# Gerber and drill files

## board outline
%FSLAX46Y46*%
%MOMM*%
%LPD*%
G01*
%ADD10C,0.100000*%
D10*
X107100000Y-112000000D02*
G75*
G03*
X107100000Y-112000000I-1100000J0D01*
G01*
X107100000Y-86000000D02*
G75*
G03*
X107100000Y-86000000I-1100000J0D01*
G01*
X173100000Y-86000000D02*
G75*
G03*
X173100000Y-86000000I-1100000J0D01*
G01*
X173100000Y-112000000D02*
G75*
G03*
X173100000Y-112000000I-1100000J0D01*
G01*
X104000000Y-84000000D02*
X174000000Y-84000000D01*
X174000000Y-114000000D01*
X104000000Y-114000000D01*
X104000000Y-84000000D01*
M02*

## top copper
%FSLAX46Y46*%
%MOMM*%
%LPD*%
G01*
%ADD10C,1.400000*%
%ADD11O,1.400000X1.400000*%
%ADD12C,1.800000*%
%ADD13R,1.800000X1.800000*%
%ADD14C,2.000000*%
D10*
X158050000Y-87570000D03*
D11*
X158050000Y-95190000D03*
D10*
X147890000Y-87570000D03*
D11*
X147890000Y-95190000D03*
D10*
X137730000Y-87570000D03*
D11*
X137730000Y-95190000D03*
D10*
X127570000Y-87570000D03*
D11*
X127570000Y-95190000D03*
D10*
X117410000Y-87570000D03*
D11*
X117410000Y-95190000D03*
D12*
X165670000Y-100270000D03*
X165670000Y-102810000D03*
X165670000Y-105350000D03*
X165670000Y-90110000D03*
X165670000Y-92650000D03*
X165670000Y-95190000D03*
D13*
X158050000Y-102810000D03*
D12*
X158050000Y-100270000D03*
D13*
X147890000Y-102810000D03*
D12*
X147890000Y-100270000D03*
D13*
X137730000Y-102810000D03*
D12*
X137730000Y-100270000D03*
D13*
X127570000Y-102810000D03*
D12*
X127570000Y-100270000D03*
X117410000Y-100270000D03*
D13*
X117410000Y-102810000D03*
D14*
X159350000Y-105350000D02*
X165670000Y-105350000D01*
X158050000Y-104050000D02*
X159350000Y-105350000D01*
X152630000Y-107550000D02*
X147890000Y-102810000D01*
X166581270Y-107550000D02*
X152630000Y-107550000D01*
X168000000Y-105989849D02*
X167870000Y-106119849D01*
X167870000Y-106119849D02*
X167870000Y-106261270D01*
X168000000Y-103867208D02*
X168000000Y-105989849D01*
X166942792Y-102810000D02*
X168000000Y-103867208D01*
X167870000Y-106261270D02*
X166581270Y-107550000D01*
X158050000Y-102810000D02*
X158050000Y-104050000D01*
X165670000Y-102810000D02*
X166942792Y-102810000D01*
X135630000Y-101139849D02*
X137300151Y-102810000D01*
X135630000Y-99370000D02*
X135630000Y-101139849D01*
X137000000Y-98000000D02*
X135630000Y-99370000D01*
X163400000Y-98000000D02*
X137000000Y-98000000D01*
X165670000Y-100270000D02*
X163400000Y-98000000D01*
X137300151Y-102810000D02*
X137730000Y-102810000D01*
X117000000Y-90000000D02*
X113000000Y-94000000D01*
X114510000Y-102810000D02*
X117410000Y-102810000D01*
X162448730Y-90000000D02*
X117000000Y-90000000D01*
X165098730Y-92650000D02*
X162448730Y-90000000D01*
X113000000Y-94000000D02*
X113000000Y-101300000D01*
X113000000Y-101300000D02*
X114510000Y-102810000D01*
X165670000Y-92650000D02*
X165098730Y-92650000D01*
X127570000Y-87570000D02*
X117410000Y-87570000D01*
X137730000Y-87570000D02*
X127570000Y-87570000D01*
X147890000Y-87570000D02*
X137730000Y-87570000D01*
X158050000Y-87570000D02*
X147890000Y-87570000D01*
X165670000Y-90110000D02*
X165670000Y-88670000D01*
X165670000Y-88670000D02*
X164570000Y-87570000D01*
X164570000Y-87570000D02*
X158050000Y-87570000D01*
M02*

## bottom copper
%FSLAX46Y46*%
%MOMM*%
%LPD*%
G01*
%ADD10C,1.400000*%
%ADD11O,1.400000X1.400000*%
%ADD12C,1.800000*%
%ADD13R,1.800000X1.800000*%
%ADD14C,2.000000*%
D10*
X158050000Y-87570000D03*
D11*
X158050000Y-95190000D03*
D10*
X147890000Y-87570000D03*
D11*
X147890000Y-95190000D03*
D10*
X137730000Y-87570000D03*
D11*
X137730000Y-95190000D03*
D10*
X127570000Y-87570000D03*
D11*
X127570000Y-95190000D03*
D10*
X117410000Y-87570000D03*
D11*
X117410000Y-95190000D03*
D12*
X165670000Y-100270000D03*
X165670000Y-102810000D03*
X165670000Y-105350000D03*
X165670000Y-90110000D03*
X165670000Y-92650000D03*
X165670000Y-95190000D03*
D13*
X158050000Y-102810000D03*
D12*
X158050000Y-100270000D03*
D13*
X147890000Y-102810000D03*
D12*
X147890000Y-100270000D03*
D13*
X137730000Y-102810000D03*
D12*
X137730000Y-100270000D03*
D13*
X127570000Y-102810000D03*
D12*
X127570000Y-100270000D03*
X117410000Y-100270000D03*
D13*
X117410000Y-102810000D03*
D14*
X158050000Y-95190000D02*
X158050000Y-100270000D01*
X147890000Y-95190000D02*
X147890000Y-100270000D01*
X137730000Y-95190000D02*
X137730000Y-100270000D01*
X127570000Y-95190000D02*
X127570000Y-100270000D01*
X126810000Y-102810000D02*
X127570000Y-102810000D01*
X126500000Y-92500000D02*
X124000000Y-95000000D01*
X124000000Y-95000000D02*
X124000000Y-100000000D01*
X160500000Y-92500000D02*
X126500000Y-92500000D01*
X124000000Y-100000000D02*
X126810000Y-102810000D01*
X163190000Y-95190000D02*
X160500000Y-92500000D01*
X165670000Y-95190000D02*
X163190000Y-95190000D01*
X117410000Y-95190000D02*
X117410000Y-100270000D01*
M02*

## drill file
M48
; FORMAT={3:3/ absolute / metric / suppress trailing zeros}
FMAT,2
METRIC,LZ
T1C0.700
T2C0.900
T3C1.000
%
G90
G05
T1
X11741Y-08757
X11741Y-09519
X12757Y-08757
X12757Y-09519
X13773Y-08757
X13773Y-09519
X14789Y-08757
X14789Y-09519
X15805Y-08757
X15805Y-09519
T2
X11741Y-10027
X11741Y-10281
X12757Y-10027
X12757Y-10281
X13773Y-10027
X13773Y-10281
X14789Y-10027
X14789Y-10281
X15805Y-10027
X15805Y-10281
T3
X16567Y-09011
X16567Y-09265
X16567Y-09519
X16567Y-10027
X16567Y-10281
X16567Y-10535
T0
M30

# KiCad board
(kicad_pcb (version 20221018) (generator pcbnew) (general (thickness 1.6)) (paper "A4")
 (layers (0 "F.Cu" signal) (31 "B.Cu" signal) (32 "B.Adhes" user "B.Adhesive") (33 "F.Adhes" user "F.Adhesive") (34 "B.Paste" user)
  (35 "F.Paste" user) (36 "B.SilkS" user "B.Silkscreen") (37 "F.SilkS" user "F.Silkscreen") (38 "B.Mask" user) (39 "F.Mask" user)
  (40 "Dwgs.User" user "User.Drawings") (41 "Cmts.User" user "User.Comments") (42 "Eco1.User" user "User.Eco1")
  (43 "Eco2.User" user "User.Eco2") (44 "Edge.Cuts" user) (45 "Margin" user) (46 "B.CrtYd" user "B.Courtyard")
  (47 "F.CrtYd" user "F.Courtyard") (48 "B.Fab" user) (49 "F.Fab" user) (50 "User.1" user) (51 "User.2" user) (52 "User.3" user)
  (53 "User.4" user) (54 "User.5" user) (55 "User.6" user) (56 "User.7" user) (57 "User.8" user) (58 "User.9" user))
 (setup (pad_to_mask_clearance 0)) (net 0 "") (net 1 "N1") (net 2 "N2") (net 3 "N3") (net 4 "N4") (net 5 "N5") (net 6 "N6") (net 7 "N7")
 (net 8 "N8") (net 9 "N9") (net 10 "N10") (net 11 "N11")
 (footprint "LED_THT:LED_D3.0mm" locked (layer "F.Cu") (at 117.41 102.81 90)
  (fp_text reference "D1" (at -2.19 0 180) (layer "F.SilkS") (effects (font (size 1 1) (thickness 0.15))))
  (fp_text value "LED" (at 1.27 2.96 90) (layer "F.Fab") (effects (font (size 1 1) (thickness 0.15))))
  (pad "1" thru_hole rect locked (at 0 0 90) (size 1.8 1.8) (drill 0.9) (layers "*.Cu" "*.Mask") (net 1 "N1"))
  (pad "2" thru_hole circle locked (at 2.54 0 90) (size 1.8 1.8) (drill 0.9) (layers "*.Cu" "*.Mask") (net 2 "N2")))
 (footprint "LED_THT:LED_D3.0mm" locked (layer "F.Cu") (at 158.05 102.81 90)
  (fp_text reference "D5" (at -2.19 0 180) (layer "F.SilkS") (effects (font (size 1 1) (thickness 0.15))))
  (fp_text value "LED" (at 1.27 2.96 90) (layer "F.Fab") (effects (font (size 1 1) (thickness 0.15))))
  (pad "1" thru_hole rect locked (at 0 0 90) (size 1.8 1.8) (drill 0.9) (layers "*.Cu" "*.Mask") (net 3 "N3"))
  (pad "2" thru_hole circle locked (at 2.54 0 90) (size 1.8 1.8) (drill 0.9) (layers "*.Cu" "*.Mask") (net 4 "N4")))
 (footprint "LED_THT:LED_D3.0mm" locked (layer "F.Cu") (at 127.57 102.81 90)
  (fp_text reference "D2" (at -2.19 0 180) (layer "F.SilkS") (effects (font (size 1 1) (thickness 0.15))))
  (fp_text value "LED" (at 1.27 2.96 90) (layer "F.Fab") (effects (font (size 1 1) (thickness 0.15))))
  (pad "1" thru_hole rect locked (at 0 0 90) (size 1.8 1.8) (drill 0.9) (layers "*.Cu" "*.Mask") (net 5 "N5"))
  (pad "2" thru_hole circle locked (at 2.54 0 90) (size 1.8 1.8) (drill 0.9) (layers "*.Cu" "*.Mask") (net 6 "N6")))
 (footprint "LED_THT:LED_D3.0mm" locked (layer "F.Cu") (at 137.73 102.81 90)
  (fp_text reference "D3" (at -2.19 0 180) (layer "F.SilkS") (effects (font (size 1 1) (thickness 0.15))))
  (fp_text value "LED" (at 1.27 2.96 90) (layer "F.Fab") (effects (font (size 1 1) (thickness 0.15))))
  (pad "1" thru_hole rect locked (at 0 0 90) (size 1.8 1.8) (drill 0.9) (layers "*.Cu" "*.Mask") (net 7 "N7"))
  (pad "2" thru_hole circle locked (at 2.54 0 90) (size 1.8 1.8) (drill 0.9) (layers "*.Cu" "*.Mask") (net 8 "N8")))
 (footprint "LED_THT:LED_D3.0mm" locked (layer "F.Cu") (at 147.89 102.81 90)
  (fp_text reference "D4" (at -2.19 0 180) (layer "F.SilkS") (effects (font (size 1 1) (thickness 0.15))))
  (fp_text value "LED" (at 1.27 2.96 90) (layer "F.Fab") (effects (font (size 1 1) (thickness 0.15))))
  (pad "1" thru_hole rect locked (at 0 0 90) (size 1.8 1.8) (drill 0.9) (layers "*.Cu" "*.Mask") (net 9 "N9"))
  (pad "2" thru_hole circle locked (at 2.54 0 90) (size 1.8 1.8) (drill 0.9) (layers "*.Cu" "*.Mask") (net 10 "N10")))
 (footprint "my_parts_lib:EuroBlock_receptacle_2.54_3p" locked (layer "B.Cu") (at 165.67 102.81 90)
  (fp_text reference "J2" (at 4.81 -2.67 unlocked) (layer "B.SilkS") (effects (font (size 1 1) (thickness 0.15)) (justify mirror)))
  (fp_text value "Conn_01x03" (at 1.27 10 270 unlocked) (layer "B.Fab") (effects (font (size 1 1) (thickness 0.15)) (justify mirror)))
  (pad "1" thru_hole circle locked (at 2.54 0 90) (size 1.8 1.8) (drill 1) (layers "*.Cu" "*.Mask") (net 7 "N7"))
  (pad "2" thru_hole circle locked (at 0 0 90) (size 1.8 1.8) (drill 1) (layers "*.Cu" "*.Mask") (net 9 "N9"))
  (pad "3" thru_hole circle locked (at -2.54 0 90) (size 1.8 1.8) (drill 1) (layers "*.Cu" "*.Mask") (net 3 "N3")))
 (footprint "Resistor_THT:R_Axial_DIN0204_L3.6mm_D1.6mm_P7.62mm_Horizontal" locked (layer "B.Cu") (at 147.89 87.57 -90)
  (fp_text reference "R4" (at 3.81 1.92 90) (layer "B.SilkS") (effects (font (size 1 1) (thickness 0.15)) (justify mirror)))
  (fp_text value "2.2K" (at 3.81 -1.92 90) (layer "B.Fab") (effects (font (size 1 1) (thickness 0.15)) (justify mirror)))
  (pad "1" thru_hole circle locked (at 0 0 270) (size 1.4 1.4) (drill 0.7) (layers "*.Cu" "*.Mask") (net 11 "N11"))
  (pad "2" thru_hole oval locked (at 7.62 0 270) (size 1.4 1.4) (drill 0.7) (layers "*.Cu" "*.Mask") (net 10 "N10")))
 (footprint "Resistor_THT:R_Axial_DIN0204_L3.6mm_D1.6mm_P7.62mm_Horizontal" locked (layer "B.Cu") (at 127.57 87.57 -90)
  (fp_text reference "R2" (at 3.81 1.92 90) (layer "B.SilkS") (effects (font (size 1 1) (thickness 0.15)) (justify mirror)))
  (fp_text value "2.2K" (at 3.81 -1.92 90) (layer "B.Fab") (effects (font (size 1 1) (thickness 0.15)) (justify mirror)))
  (pad "1" thru_hole circle locked (at 0 0 270) (size 1.4 1.4) (drill 0.7) (layers "*.Cu" "*.Mask") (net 11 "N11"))
  (pad "2" thru_hole oval locked (at 7.62 0 270) (size 1.4 1.4) (drill 0.7) (layers "*.Cu" "*.Mask") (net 6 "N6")))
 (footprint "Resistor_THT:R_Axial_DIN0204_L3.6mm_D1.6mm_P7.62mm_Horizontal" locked (layer "B.Cu") (at 158.05 87.57 -90)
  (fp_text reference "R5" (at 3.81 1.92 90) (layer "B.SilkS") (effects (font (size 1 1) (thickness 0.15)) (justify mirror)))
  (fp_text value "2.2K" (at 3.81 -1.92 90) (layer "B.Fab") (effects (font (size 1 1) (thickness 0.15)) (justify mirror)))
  (pad "1" thru_hole circle locked (at 0 0 270) (size 1.4 1.4) (drill 0.7) (layers "*.Cu" "*.Mask") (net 11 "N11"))
  (pad "2" thru_hole oval locked (at 7.62 0 270) (size 1.4 1.4) (drill 0.7) (layers "*.Cu" "*.Mask") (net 4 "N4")))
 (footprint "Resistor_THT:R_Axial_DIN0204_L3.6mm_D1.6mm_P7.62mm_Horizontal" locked (layer "B.Cu") (at 117.41 87.57 -90)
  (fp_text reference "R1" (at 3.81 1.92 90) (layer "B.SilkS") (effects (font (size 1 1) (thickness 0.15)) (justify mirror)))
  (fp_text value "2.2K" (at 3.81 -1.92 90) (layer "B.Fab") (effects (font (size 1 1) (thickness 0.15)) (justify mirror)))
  (pad "1" thru_hole circle locked (at 0 0 270) (size 1.4 1.4) (drill 0.7) (layers "*.Cu" "*.Mask") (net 11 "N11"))
  (pad "2" thru_hole oval locked (at 7.62 0 270) (size 1.4 1.4) (drill 0.7) (layers "*.Cu" "*.Mask") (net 2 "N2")))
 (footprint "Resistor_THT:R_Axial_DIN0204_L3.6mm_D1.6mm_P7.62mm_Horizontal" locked (layer "B.Cu") (at 137.73 87.57 -90)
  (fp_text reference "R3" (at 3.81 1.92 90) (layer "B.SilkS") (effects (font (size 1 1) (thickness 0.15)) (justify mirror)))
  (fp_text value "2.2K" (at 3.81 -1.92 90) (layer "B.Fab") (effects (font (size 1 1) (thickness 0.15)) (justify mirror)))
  (pad "1" thru_hole circle locked (at 0 0 270) (size 1.4 1.4) (drill 0.7) (layers "*.Cu" "*.Mask") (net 11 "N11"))
  (pad "2" thru_hole oval locked (at 7.62 0 270) (size 1.4 1.4) (drill 0.7) (layers "*.Cu" "*.Mask") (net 8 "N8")))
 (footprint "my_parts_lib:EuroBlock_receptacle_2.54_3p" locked (layer "B.Cu") (at 165.67 92.65 90)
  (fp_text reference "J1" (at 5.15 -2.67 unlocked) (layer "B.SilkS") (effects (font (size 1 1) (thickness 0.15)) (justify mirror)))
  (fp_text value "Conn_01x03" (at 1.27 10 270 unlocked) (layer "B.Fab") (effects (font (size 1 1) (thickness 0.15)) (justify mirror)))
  (pad "1" thru_hole circle locked (at 2.54 0 90) (size 1.8 1.8) (drill 1) (layers "*.Cu" "*.Mask") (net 11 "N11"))
  (pad "2" thru_hole circle locked (at 0 0 90) (size 1.8 1.8) (drill 1) (layers "*.Cu" "*.Mask") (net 1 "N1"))
  (pad "3" thru_hole circle locked (at -2.54 0 90) (size 1.8 1.8) (drill 1) (layers "*.Cu" "*.Mask") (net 5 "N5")))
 (gr_rect locked (start 104 84) (end 174 114) (stroke (width 0.1) (type default)) (fill none) (layer "Edge.Cuts"))
 (gr_circle locked (center 106 86) (end 107.1 86) (stroke (width 0.1) (type default)) (fill none) (layer "Edge.Cuts"))
 (gr_circle locked (center 172 112) (end 173.1 112) (stroke (width 0.1) (type default)) (fill none) (layer "Edge.Cuts"))
 (gr_circle locked (center 172 86) (end 173.1 86) (stroke (width 0.1) (type default)) (fill none) (layer "Edge.Cuts"))
 (gr_circle locked (center 106 112) (end 107.1 112) (stroke (width 0.1) (type default)) (fill none) (layer "Edge.Cuts"))
 (segment (start 165.09873 92.65) (end 162.44873 90) (width 2) (layer "F.Cu") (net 1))
 (segment (start 162.44873 90) (end 117 90) (width 2) (layer "F.Cu") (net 1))
 (segment (start 165.67 92.65) (end 165.09873 92.65) (width 2) (layer "F.Cu") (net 1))
 (segment (start 117 90) (end 113 94) (width 2) (layer "F.Cu") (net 1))
 (segment (start 113 94) (end 113 101.3) (width 2) (layer "F.Cu") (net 1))
 (segment (start 114.51 102.81) (end 117.41 102.81) (width 2) (layer "F.Cu") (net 1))
 (segment (start 113 101.3) (end 114.51 102.81) (width 2) (layer "F.Cu") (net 1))
 (segment (start 117.41 95.19) (end 117.41 100.27) (width 2) (layer "B.Cu") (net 2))
 (segment (start 126.5 92.5) (end 124 95) (width 2) (layer "B.Cu") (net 5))
 (segment (start 124 95) (end 124 100) (width 2) (layer "B.Cu") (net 5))
 (segment (start 126.81 102.81) (end 127.57 102.81) (width 2) (layer "B.Cu") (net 5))
 (segment (start 160.5 92.5) (end 126.5 92.5) (width 2) (layer "B.Cu") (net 5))
 (segment (start 124 100) (end 126.81 102.81) (width 2) (layer "B.Cu") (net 5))
 (segment (start 163.19 95.19) (end 160.5 92.5) (width 2) (layer "B.Cu") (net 5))
 (segment (start 165.67 95.19) (end 163.19 95.19) (width 2) (layer "B.Cu") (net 5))
 (segment (start 127.57 95.19) (end 127.57 100.27) (width 2) (layer "B.Cu") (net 6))
 (segment (start 163.4 98) (end 137 98) (width 2) (layer "F.Cu") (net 7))
 (segment (start 137.300151 102.81) (end 137.73 102.81) (width 2) (layer "F.Cu") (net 7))
 (segment (start 137 98) (end 135.63 99.37) (width 2) (layer "F.Cu") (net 7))
 (segment (start 135.63 99.37) (end 135.63 101.139849) (width 2) (layer "F.Cu") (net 7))
 (segment (start 165.67 100.27) (end 163.4 98) (width 2) (layer "F.Cu") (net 7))
 (segment (start 135.63 101.139849) (end 137.300151 102.81) (width 2) (layer "F.Cu") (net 7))
 (segment (start 137.73 95.19) (end 137.73 100.27) (width 2) (layer "B.Cu") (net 8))
 (segment (start 165.67 102.81) (end 166.942792 102.81) (width 2) (layer "F.Cu") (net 9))
 (segment (start 167.87 106.26127) (end 166.58127 107.55) (width 2) (layer "F.Cu") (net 9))
 (segment (start 168 103.867208) (end 168 105.989849) (width 2) (layer "F.Cu") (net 9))
 (segment (start 152.63 107.55) (end 147.89 102.81) (width 2) (layer "F.Cu") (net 9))
 (segment (start 166.942792 102.81) (end 168 103.867208) (width 2) (layer "F.Cu") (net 9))
 (segment (start 168 105.989849) (end 167.87 106.119849) (width 2) (layer "F.Cu") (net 9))
 (segment (start 167.87 106.119849) (end 167.87 106.26127) (width 2) (layer "F.Cu") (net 9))
 (segment (start 166.58127 107.55) (end 152.63 107.55) (width 2) (layer "F.Cu") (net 9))
 (segment (start 147.89 95.19) (end 147.89 100.27) (width 2) (layer "B.Cu") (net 10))
 (segment (start 158.05 102.81) (end 158.05 104.05) (width 2) (layer "F.Cu") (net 3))
 (segment (start 159.35 105.35) (end 165.67 105.35) (width 2) (layer "F.Cu") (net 3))
 (segment (start 158.05 104.05) (end 159.35 105.35) (width 2) (layer "F.Cu") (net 3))
 (segment (start 158.05 95.19) (end 158.05 100.27) (width 2) (layer "B.Cu") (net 4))
 (segment (start 165.67 90.11) (end 165.67 88.67) (width 2) (layer "F.Cu") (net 11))
 (segment (start 158.05 87.57) (end 147.89 87.57) (width 2) (layer "F.Cu") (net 11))
 (segment (start 127.57 87.57) (end 117.41 87.57) (width 2) (layer "F.Cu") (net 11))
 (segment (start 165.67 88.67) (end 164.57 87.57) (width 2) (layer "F.Cu") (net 11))
 (segment (start 147.89 87.57) (end 137.73 87.57) (width 2) (layer "F.Cu") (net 11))
 (segment (start 164.57 87.57) (end 158.05 87.57) (width 2) (layer "F.Cu") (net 11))
 (segment (start 137.73 87.57) (end 127.57 87.57) (width 2) (layer "F.Cu") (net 11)))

